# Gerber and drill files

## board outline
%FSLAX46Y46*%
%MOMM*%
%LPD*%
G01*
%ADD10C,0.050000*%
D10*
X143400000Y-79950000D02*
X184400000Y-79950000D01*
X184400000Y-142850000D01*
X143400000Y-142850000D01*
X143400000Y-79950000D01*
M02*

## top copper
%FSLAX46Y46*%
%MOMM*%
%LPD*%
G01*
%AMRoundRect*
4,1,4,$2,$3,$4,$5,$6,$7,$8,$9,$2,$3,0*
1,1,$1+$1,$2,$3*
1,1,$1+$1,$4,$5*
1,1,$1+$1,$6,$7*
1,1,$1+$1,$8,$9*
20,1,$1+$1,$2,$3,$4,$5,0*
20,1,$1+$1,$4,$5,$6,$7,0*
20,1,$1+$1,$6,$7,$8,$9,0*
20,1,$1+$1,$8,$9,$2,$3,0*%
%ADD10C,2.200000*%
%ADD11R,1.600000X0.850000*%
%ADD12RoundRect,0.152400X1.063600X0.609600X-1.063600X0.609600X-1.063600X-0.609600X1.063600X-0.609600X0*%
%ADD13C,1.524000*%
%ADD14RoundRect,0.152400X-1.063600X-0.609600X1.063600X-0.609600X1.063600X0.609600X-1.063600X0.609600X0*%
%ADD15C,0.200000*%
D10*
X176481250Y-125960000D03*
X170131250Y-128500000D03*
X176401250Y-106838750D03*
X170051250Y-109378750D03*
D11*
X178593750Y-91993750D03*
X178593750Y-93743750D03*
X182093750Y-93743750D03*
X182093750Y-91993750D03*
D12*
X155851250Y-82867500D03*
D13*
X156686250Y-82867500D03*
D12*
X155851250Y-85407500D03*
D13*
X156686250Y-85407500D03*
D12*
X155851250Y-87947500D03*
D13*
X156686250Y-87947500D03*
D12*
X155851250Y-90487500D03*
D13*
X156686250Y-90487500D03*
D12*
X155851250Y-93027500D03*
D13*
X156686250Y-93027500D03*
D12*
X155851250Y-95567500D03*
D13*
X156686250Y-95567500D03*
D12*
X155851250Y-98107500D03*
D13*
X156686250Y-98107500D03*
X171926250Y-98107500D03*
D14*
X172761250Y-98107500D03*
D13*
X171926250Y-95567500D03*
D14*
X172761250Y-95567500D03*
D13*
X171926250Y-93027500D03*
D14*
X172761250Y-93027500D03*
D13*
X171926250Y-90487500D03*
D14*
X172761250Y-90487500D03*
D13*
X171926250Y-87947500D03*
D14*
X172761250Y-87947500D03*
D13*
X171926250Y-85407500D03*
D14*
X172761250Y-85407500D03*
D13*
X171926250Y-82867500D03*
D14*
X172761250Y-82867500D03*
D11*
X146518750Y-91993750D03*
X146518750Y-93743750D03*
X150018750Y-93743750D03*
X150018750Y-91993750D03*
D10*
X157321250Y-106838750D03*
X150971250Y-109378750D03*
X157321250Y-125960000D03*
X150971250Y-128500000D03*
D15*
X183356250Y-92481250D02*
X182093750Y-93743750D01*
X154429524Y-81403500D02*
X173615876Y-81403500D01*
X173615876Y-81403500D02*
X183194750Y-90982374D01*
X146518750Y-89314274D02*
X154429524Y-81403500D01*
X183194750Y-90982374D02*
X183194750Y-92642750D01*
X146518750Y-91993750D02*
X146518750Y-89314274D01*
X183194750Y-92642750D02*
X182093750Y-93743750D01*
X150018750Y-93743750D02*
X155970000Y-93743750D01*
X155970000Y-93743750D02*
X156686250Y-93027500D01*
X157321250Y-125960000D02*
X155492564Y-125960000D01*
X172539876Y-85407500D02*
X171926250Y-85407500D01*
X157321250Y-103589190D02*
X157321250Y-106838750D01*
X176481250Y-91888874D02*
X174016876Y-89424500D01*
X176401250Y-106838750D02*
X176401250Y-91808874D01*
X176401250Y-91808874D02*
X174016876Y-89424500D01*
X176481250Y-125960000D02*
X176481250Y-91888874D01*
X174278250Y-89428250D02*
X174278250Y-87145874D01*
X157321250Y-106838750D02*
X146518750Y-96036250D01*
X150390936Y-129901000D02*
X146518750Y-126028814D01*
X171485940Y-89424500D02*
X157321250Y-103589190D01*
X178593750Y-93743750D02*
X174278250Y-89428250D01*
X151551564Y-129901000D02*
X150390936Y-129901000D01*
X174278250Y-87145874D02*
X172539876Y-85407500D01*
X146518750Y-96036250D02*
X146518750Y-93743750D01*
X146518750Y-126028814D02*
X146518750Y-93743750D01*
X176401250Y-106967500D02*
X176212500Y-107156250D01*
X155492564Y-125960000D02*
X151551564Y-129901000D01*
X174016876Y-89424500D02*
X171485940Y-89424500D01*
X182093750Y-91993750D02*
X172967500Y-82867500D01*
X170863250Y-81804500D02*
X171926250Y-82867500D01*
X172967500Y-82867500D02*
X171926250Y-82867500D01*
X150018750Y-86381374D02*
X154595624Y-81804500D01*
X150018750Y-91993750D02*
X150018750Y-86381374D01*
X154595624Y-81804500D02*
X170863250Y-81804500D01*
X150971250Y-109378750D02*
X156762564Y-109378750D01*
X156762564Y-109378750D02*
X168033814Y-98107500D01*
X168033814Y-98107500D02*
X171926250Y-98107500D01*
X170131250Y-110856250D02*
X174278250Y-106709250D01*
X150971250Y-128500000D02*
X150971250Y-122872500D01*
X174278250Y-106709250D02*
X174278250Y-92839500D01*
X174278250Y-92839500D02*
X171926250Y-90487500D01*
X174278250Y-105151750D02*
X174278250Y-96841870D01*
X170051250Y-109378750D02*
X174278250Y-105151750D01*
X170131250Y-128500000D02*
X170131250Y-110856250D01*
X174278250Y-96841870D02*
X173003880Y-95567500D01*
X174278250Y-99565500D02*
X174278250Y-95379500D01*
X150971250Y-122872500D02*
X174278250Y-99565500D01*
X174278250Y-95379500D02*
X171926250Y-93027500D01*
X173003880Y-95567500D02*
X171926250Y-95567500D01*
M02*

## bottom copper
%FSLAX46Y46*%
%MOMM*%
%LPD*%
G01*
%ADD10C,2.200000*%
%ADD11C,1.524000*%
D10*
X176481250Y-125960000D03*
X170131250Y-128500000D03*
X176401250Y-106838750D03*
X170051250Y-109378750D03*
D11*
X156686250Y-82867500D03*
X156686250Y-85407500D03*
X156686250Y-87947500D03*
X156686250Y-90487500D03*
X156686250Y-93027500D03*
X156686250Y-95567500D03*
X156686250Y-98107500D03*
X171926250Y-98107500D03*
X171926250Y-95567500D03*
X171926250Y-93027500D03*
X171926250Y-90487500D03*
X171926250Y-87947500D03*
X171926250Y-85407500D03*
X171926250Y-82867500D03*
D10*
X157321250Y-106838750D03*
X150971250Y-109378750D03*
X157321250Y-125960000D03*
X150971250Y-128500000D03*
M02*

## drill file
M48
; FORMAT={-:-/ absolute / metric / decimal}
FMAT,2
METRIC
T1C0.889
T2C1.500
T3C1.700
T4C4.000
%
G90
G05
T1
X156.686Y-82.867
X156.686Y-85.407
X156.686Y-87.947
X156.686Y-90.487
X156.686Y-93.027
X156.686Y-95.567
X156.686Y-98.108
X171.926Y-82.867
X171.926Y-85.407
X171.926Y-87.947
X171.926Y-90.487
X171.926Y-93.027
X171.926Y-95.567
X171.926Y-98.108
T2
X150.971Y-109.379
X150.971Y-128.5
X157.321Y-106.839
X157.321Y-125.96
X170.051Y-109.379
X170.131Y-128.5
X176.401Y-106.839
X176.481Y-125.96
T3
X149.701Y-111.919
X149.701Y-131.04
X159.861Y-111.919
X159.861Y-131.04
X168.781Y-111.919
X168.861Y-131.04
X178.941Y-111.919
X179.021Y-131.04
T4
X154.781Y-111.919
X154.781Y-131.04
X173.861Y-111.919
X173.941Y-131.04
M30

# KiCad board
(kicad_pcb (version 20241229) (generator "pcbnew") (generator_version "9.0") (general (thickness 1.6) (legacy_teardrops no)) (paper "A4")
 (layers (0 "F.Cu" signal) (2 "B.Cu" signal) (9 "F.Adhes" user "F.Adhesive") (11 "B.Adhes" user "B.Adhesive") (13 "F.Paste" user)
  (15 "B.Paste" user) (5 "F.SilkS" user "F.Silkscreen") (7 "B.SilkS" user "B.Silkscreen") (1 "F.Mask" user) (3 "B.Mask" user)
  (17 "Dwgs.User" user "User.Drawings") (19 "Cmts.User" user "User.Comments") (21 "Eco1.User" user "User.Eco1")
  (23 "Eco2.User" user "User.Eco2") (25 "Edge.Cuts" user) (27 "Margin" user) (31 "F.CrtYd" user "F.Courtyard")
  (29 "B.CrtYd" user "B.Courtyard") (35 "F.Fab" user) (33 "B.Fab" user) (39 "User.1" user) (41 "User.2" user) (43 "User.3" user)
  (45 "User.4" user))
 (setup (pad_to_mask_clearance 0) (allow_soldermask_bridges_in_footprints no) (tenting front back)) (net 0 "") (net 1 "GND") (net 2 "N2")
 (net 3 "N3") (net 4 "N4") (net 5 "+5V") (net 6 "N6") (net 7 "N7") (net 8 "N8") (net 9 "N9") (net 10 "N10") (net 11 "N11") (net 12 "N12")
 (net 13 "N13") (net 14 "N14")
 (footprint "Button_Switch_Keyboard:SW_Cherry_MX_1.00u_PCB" (layer "F.Cu") (at 176.48125 125.96)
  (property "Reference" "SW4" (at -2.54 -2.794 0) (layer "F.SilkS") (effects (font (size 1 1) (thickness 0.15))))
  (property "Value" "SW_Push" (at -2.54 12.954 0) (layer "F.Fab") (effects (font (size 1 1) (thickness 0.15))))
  (pad "" np_thru_hole circle (at -7.62 5.08) (size 1.7 1.7) (drill 1.7) (layers "*.Cu" "*.Mask"))
  (pad "" np_thru_hole circle (at -2.54 5.08) (size 4 4) (drill 4) (layers "*.Cu" "*.Mask"))
  (pad "" np_thru_hole circle (at 2.54 5.08) (size 1.7 1.7) (drill 1.7) (layers "*.Cu" "*.Mask"))
  (pad "1" thru_hole circle (at 0 0) (size 2.2 2.2) (drill 1.5) (layers "*.Cu" "*.Mask") (remove_unused_layers no) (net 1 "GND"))
  (pad "2" thru_hole circle (at -6.35 2.54) (size 2.2 2.2) (drill 1.5) (layers "*.Cu" "*.Mask") (remove_unused_layers no) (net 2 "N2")))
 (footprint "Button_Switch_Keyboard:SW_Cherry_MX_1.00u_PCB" (layer "F.Cu") (at 176.40125 106.83875)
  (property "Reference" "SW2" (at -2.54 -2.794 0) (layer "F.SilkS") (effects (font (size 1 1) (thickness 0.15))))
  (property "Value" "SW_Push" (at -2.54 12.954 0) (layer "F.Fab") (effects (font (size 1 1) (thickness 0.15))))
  (pad "" np_thru_hole circle (at -7.62 5.08) (size 1.7 1.7) (drill 1.7) (layers "*.Cu" "*.Mask"))
  (pad "" np_thru_hole circle (at -2.54 5.08) (size 4 4) (drill 4) (layers "*.Cu" "*.Mask"))
  (pad "" np_thru_hole circle (at 2.54 5.08) (size 1.7 1.7) (drill 1.7) (layers "*.Cu" "*.Mask"))
  (pad "1" thru_hole circle (at 0 0) (size 2.2 2.2) (drill 1.5) (layers "*.Cu" "*.Mask") (remove_unused_layers no) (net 1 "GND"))
  (pad "2" thru_hole circle (at -6.35 2.54) (size 2.2 2.2) (drill 1.5) (layers "*.Cu" "*.Mask") (remove_unused_layers no) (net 2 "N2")))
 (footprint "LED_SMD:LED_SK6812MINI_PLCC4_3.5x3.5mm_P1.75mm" (layer "F.Cu") (at 180.34375 92.86875)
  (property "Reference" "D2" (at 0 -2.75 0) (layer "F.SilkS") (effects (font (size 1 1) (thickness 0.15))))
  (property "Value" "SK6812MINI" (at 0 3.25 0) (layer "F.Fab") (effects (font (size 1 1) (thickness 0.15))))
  (pad "1" smd rect (at -1.75 -0.875) (size 1.6 0.85) (layers "F.Cu" "F.Mask" "F.Paste") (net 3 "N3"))
  (pad "2" smd rect (at -1.75 0.875) (size 1.6 0.85) (layers "F.Cu" "F.Mask" "F.Paste") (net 1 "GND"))
  (pad "3" smd rect (at 1.75 0.875) (size 1.6 0.85) (layers "F.Cu" "F.Mask" "F.Paste") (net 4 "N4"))
  (pad "4" smd rect (at 1.75 -0.875) (size 1.6 0.85) (layers "F.Cu" "F.Mask" "F.Paste") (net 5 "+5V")))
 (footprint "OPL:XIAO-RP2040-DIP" (layer "F.Cu") (at 164.30625 90.4875)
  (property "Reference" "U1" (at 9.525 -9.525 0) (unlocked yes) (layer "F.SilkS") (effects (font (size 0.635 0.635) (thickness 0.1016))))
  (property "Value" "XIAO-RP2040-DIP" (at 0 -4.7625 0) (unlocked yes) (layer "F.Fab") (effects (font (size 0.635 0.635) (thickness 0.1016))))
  (pad "1" smd roundrect (at -8.455 -7.62 180) (size 2.432 1.524) (layers "F.Cu" "F.Mask") (roundrect_rratio 0.1) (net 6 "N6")
   (thermal_bridge_angle 45))
  (pad "1" thru_hole circle (at -7.62 -7.62 180) (size 1.524 1.524) (drill 0.889) (layers "*.Cu" "*.Mask") (remove_unused_layers no)
   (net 6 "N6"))
  (pad "2" smd roundrect (at -8.455 -5.08 180) (size 2.432 1.524) (layers "F.Cu" "F.Mask") (roundrect_rratio 0.1) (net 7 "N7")
   (thermal_bridge_angle 45))
  (pad "2" thru_hole circle (at -7.62 -5.08 180) (size 1.524 1.524) (drill 0.889) (layers "*.Cu" "*.Mask") (remove_unused_layers no)
   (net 7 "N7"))
  (pad "3" smd roundrect (at -8.455 -2.54 180) (size 2.432 1.524) (layers "F.Cu" "F.Mask") (roundrect_rratio 0.1) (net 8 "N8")
   (thermal_bridge_angle 45))
  (pad "3" thru_hole circle (at -7.62 -2.54 180) (size 1.524 1.524) (drill 0.889) (layers "*.Cu" "*.Mask") (remove_unused_layers no)
   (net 8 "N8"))
  (pad "4" smd roundrect (at -8.455 0 180) (size 2.432 1.524) (layers "F.Cu" "F.Mask") (roundrect_rratio 0.1) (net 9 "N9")
   (thermal_bridge_angle 45))
  (pad "4" thru_hole circle (at -7.62 0 180) (size 1.524 1.524) (drill 0.889) (layers "*.Cu" "*.Mask") (remove_unused_layers no)
   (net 9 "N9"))
  (pad "5" smd roundrect (at -8.455 2.54 180) (size 2.432 1.524) (layers "F.Cu" "F.Mask") (roundrect_rratio 0.1) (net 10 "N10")
   (thermal_bridge_angle 45))
  (pad "5" thru_hole circle (at -7.62 2.54 180) (size 1.524 1.524) (drill 0.889) (layers "*.Cu" "*.Mask") (remove_unused_layers no)
   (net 10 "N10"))
  (pad "6" smd roundrect (at -8.455 5.08 180) (size 2.432 1.524) (layers "F.Cu" "F.Mask") (roundrect_rratio 0.1) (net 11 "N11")
   (thermal_bridge_angle 45))
  (pad "6" thru_hole circle (at -7.62 5.08 180) (size 1.524 1.524) (drill 0.889) (layers "*.Cu" "*.Mask") (remove_unused_layers no)
   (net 11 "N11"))
  (pad "7" smd roundrect (at -8.455 7.62 180) (size 2.432 1.524) (layers "F.Cu" "F.Mask") (roundrect_rratio 0.1) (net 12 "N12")
   (thermal_bridge_angle 45))
  (pad "7" thru_hole circle (at -7.62 7.62 180) (size 1.524 1.524) (drill 0.889) (layers "*.Cu" "*.Mask") (remove_unused_layers no)
   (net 12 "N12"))
  (pad "8" thru_hole circle (at 7.62 7.62) (size 1.524 1.524) (drill 0.889) (layers "*.Cu" "*.Mask") (remove_unused_layers no)
   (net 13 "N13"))
  (pad "8" smd roundrect (at 8.455 7.62) (size 2.432 1.524) (layers "F.Cu" "F.Mask") (roundrect_rratio 0.1) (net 13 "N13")
   (thermal_bridge_angle 45))
  (pad "9" thru_hole circle (at 7.62 5.08) (size 1.524 1.524) (drill 0.889) (layers "*.Cu" "*.Mask") (remove_unused_layers no) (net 2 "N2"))
  (pad "9" smd roundrect (at 8.455 5.08) (size 2.432 1.524) (layers "F.Cu" "F.Mask") (roundrect_rratio 0.1) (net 2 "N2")
   (thermal_bridge_angle 45))
  (pad "10" thru_hole circle (at 7.62 2.54) (size 1.524 1.524) (drill 0.889) (layers "*.Cu" "*.Mask") (remove_unused_layers no) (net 2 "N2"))
  (pad "10" smd roundrect (at 8.455 2.54) (size 2.432 1.524) (layers "F.Cu" "F.Mask") (roundrect_rratio 0.1) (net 2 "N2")
   (thermal_bridge_angle 45))
  (pad "11" thru_hole circle (at 7.62 0) (size 1.524 1.524) (drill 0.889) (layers "*.Cu" "*.Mask") (remove_unused_layers no) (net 2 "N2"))
  (pad "11" smd roundrect (at 8.455 0) (size 2.432 1.524) (layers "F.Cu" "F.Mask") (roundrect_rratio 0.1) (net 2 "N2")
   (thermal_bridge_angle 45))
  (pad "12" thru_hole circle (at 7.62 -2.54) (size 1.524 1.524) (drill 0.889) (layers "*.Cu" "*.Mask") (remove_unused_layers no)
   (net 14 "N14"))
  (pad "12" smd roundrect (at 8.455 -2.54) (size 2.432 1.524) (layers "F.Cu" "F.Mask") (roundrect_rratio 0.1) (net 14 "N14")
   (thermal_bridge_angle 45))
  (pad "13" thru_hole circle (at 7.62 -5.08) (size 1.524 1.524) (drill 0.889) (layers "*.Cu" "*.Mask") (remove_unused_layers no)
   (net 1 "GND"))
  (pad "13" smd roundrect (at 8.455 -5.08) (size 2.432 1.524) (layers "F.Cu" "F.Mask") (roundrect_rratio 0.1) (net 1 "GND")
   (thermal_bridge_angle 45))
  (pad "14" thru_hole circle (at 7.62 -7.62) (size 1.524 1.524) (drill 0.889) (layers "*.Cu" "*.Mask") (remove_unused_layers no)
   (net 5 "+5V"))
  (pad "14" smd roundrect (at 8.455 -7.62) (size 2.432 1.524) (layers "F.Cu" "F.Mask") (roundrect_rratio 0.1) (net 5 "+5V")
   (thermal_bridge_angle 45)))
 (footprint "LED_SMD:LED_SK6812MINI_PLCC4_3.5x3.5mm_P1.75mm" (layer "F.Cu") (at 148.26875 92.86875)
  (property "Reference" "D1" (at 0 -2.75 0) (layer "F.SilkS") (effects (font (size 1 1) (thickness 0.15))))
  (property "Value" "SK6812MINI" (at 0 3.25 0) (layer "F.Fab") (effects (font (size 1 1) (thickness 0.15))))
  (pad "1" smd rect (at -1.75 -0.875) (size 1.6 0.85) (layers "F.Cu" "F.Mask" "F.Paste") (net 4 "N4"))
  (pad "2" smd rect (at -1.75 0.875) (size 1.6 0.85) (layers "F.Cu" "F.Mask" "F.Paste") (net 1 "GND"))
  (pad "3" smd rect (at 1.75 0.875) (size 1.6 0.85) (layers "F.Cu" "F.Mask" "F.Paste") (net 10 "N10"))
  (pad "4" smd rect (at 1.75 -0.875) (size 1.6 0.85) (layers "F.Cu" "F.Mask" "F.Paste") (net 5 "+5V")))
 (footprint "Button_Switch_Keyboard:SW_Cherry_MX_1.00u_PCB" (layer "F.Cu") (at 157.32125 106.83875)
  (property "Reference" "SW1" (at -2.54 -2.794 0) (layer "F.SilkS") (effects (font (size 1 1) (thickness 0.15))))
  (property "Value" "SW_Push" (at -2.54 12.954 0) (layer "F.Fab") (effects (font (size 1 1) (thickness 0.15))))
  (pad "" np_thru_hole circle (at -7.62 5.08) (size 1.7 1.7) (drill 1.7) (layers "*.Cu" "*.Mask"))
  (pad "" np_thru_hole circle (at -2.54 5.08) (size 4 4) (drill 4) (layers "*.Cu" "*.Mask"))
  (pad "" np_thru_hole circle (at 2.54 5.08) (size 1.7 1.7) (drill 1.7) (layers "*.Cu" "*.Mask"))
  (pad "1" thru_hole circle (at 0 0) (size 2.2 2.2) (drill 1.5) (layers "*.Cu" "*.Mask") (remove_unused_layers no) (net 1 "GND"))
  (pad "2" thru_hole circle (at -6.35 2.54) (size 2.2 2.2) (drill 1.5) (layers "*.Cu" "*.Mask") (remove_unused_layers no) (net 13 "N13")))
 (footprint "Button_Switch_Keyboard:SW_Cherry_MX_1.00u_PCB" (layer "F.Cu") (at 157.32125 125.96)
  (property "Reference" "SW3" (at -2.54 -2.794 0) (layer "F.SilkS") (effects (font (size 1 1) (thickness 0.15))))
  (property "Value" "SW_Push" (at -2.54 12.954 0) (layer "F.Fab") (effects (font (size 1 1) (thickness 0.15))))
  (pad "" np_thru_hole circle (at -7.62 5.08) (size 1.7 1.7) (drill 1.7) (layers "*.Cu" "*.Mask"))
  (pad "" np_thru_hole circle (at -2.54 5.08) (size 4 4) (drill 4) (layers "*.Cu" "*.Mask"))
  (pad "" np_thru_hole circle (at 2.54 5.08) (size 1.7 1.7) (drill 1.7) (layers "*.Cu" "*.Mask"))
  (pad "1" thru_hole circle (at 0 0) (size 2.2 2.2) (drill 1.5) (layers "*.Cu" "*.Mask") (remove_unused_layers no) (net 1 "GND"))
  (pad "2" thru_hole circle (at -6.35 2.54) (size 2.2 2.2) (drill 1.5) (layers "*.Cu" "*.Mask") (remove_unused_layers no) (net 2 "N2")))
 (gr_rect (start 143.4 79.95) (end 184.4 142.85) (stroke (width 0.05) (type default)) (fill no) (layer "Edge.Cuts"))
 (segment (start 183.35625 92.48125) (end 182.09375 93.74375) (width 0.2) (layer "F.Cu") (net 4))
 (segment (start 154.429524 81.4035) (end 173.615876 81.4035) (width 0.2) (layer "F.Cu") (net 4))
 (segment (start 173.615876 81.4035) (end 183.19475 90.982374) (width 0.2) (layer "F.Cu") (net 4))
 (segment (start 146.51875 89.314274) (end 154.429524 81.4035) (width 0.2) (layer "F.Cu") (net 4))
 (segment (start 183.19475 90.982374) (end 183.19475 92.64275) (width 0.2) (layer "F.Cu") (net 4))
 (segment (start 146.51875 91.99375) (end 146.51875 89.314274) (width 0.2) (layer "F.Cu") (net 4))
 (segment (start 183.19475 92.64275) (end 182.09375 93.74375) (width 0.2) (layer "F.Cu") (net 4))
 (segment (start 150.01875 93.74375) (end 155.97 93.74375) (width 0.2) (layer "F.Cu") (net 10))
 (segment (start 155.97 93.74375) (end 156.68625 93.0275) (width 0.2) (layer "F.Cu") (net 10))
 (segment (start 157.32125 125.96) (end 155.492564 125.96) (width 0.2) (layer "F.Cu") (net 1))
 (segment (start 172.539876 85.4075) (end 171.92625 85.4075) (width 0.2) (layer "F.Cu") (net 1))
 (segment (start 157.32125 103.58919) (end 157.32125 106.83875) (width 0.2) (layer "F.Cu") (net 1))
 (segment (start 176.48125 91.888874) (end 174.016876 89.4245) (width 0.2) (layer "F.Cu") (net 1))
 (segment (start 176.40125 106.83875) (end 176.40125 91.808874) (width 0.2) (layer "F.Cu") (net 1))
 (segment (start 176.40125 91.808874) (end 174.016876 89.4245) (width 0.2) (layer "F.Cu") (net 1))
 (segment (start 176.48125 125.96) (end 176.48125 91.888874) (width 0.2) (layer "F.Cu") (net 1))
 (segment (start 174.27825 89.42825) (end 174.27825 87.145874) (width 0.2) (layer "F.Cu") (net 1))
 (segment (start 157.32125 106.83875) (end 146.51875 96.03625) (width 0.2) (layer "F.Cu") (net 1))
 (segment (start 150.390936 129.901) (end 146.51875 126.028814) (width 0.2) (layer "F.Cu") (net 1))
 (segment (start 171.48594 89.4245) (end 157.32125 103.58919) (width 0.2) (layer "F.Cu") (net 1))
 (segment (start 178.59375 93.74375) (end 174.27825 89.42825) (width 0.2) (layer "F.Cu") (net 1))
 (segment (start 151.551564 129.901) (end 150.390936 129.901) (width 0.2) (layer "F.Cu") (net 1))
 (segment (start 174.27825 87.145874) (end 172.539876 85.4075) (width 0.2) (layer "F.Cu") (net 1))
 (segment (start 146.51875 96.03625) (end 146.51875 93.74375) (width 0.2) (layer "F.Cu") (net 1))
 (segment (start 146.51875 126.028814) (end 146.51875 93.74375) (width 0.2) (layer "F.Cu") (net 1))
 (segment (start 176.40125 106.9675) (end 176.2125 107.15625) (width 0.2) (layer "F.Cu") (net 1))
 (segment (start 155.492564 125.96) (end 151.551564 129.901) (width 0.2) (layer "F.Cu") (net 1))
 (segment (start 174.016876 89.4245) (end 171.48594 89.4245) (width 0.2) (layer "F.Cu") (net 1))
 (segment (start 182.09375 91.99375) (end 172.9675 82.8675) (width 0.2) (layer "F.Cu") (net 5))
 (segment (start 170.86325 81.8045) (end 171.92625 82.8675) (width 0.2) (layer "F.Cu") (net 5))
 (segment (start 172.9675 82.8675) (end 171.92625 82.8675) (width 0.2) (layer "F.Cu") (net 5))
 (segment (start 150.01875 86.381374) (end 154.595624 81.8045) (width 0.2) (layer "F.Cu") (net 5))
 (segment (start 150.01875 91.99375) (end 150.01875 86.381374) (width 0.2) (layer "F.Cu") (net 5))
 (segment (start 154.595624 81.8045) (end 170.86325 81.8045) (width 0.2) (layer "F.Cu") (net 5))
 (segment (start 150.97125 109.37875) (end 156.762564 109.37875) (width 0.2) (layer "F.Cu") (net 13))
 (segment (start 156.762564 109.37875) (end 168.033814 98.1075) (width 0.2) (layer "F.Cu") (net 13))
 (segment (start 168.033814 98.1075) (end 171.92625 98.1075) (width 0.2) (layer "F.Cu") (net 13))
 (segment (start 170.13125 110.85625) (end 174.27825 106.70925) (width 0.2) (layer "F.Cu") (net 2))
 (segment (start 150.97125 128.5) (end 150.97125 122.8725) (width 0.2) (layer "F.Cu") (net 2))
 (segment (start 174.27825 106.70925) (end 174.27825 92.8395) (width 0.2) (layer "F.Cu") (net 2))
 (segment (start 174.27825 92.8395) (end 171.92625 90.4875) (width 0.2) (layer "F.Cu") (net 2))
 (segment (start 174.27825 105.15175) (end 174.27825 96.84187) (width 0.2) (layer "F.Cu") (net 2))
 (segment (start 170.05125 109.37875) (end 174.27825 105.15175) (width 0.2) (layer "F.Cu") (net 2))
 (segment (start 170.13125 128.5) (end 170.13125 110.85625) (width 0.2) (layer "F.Cu") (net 2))
 (segment (start 174.27825 96.84187) (end 173.00388 95.5675) (width 0.2) (layer "F.Cu") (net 2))
 (segment (start 174.27825 99.5655) (end 174.27825 95.3795) (width 0.2) (layer "F.Cu") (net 2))
 (segment (start 150.97125 122.8725) (end 174.27825 99.5655) (width 0.2) (layer "F.Cu") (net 2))
 (segment (start 174.27825 95.3795) (end 171.92625 93.0275) (width 0.2) (layer "F.Cu") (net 2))
 (segment (start 173.00388 95.5675) (end 171.92625 95.5675) (width 0.2) (layer "F.Cu") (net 2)))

